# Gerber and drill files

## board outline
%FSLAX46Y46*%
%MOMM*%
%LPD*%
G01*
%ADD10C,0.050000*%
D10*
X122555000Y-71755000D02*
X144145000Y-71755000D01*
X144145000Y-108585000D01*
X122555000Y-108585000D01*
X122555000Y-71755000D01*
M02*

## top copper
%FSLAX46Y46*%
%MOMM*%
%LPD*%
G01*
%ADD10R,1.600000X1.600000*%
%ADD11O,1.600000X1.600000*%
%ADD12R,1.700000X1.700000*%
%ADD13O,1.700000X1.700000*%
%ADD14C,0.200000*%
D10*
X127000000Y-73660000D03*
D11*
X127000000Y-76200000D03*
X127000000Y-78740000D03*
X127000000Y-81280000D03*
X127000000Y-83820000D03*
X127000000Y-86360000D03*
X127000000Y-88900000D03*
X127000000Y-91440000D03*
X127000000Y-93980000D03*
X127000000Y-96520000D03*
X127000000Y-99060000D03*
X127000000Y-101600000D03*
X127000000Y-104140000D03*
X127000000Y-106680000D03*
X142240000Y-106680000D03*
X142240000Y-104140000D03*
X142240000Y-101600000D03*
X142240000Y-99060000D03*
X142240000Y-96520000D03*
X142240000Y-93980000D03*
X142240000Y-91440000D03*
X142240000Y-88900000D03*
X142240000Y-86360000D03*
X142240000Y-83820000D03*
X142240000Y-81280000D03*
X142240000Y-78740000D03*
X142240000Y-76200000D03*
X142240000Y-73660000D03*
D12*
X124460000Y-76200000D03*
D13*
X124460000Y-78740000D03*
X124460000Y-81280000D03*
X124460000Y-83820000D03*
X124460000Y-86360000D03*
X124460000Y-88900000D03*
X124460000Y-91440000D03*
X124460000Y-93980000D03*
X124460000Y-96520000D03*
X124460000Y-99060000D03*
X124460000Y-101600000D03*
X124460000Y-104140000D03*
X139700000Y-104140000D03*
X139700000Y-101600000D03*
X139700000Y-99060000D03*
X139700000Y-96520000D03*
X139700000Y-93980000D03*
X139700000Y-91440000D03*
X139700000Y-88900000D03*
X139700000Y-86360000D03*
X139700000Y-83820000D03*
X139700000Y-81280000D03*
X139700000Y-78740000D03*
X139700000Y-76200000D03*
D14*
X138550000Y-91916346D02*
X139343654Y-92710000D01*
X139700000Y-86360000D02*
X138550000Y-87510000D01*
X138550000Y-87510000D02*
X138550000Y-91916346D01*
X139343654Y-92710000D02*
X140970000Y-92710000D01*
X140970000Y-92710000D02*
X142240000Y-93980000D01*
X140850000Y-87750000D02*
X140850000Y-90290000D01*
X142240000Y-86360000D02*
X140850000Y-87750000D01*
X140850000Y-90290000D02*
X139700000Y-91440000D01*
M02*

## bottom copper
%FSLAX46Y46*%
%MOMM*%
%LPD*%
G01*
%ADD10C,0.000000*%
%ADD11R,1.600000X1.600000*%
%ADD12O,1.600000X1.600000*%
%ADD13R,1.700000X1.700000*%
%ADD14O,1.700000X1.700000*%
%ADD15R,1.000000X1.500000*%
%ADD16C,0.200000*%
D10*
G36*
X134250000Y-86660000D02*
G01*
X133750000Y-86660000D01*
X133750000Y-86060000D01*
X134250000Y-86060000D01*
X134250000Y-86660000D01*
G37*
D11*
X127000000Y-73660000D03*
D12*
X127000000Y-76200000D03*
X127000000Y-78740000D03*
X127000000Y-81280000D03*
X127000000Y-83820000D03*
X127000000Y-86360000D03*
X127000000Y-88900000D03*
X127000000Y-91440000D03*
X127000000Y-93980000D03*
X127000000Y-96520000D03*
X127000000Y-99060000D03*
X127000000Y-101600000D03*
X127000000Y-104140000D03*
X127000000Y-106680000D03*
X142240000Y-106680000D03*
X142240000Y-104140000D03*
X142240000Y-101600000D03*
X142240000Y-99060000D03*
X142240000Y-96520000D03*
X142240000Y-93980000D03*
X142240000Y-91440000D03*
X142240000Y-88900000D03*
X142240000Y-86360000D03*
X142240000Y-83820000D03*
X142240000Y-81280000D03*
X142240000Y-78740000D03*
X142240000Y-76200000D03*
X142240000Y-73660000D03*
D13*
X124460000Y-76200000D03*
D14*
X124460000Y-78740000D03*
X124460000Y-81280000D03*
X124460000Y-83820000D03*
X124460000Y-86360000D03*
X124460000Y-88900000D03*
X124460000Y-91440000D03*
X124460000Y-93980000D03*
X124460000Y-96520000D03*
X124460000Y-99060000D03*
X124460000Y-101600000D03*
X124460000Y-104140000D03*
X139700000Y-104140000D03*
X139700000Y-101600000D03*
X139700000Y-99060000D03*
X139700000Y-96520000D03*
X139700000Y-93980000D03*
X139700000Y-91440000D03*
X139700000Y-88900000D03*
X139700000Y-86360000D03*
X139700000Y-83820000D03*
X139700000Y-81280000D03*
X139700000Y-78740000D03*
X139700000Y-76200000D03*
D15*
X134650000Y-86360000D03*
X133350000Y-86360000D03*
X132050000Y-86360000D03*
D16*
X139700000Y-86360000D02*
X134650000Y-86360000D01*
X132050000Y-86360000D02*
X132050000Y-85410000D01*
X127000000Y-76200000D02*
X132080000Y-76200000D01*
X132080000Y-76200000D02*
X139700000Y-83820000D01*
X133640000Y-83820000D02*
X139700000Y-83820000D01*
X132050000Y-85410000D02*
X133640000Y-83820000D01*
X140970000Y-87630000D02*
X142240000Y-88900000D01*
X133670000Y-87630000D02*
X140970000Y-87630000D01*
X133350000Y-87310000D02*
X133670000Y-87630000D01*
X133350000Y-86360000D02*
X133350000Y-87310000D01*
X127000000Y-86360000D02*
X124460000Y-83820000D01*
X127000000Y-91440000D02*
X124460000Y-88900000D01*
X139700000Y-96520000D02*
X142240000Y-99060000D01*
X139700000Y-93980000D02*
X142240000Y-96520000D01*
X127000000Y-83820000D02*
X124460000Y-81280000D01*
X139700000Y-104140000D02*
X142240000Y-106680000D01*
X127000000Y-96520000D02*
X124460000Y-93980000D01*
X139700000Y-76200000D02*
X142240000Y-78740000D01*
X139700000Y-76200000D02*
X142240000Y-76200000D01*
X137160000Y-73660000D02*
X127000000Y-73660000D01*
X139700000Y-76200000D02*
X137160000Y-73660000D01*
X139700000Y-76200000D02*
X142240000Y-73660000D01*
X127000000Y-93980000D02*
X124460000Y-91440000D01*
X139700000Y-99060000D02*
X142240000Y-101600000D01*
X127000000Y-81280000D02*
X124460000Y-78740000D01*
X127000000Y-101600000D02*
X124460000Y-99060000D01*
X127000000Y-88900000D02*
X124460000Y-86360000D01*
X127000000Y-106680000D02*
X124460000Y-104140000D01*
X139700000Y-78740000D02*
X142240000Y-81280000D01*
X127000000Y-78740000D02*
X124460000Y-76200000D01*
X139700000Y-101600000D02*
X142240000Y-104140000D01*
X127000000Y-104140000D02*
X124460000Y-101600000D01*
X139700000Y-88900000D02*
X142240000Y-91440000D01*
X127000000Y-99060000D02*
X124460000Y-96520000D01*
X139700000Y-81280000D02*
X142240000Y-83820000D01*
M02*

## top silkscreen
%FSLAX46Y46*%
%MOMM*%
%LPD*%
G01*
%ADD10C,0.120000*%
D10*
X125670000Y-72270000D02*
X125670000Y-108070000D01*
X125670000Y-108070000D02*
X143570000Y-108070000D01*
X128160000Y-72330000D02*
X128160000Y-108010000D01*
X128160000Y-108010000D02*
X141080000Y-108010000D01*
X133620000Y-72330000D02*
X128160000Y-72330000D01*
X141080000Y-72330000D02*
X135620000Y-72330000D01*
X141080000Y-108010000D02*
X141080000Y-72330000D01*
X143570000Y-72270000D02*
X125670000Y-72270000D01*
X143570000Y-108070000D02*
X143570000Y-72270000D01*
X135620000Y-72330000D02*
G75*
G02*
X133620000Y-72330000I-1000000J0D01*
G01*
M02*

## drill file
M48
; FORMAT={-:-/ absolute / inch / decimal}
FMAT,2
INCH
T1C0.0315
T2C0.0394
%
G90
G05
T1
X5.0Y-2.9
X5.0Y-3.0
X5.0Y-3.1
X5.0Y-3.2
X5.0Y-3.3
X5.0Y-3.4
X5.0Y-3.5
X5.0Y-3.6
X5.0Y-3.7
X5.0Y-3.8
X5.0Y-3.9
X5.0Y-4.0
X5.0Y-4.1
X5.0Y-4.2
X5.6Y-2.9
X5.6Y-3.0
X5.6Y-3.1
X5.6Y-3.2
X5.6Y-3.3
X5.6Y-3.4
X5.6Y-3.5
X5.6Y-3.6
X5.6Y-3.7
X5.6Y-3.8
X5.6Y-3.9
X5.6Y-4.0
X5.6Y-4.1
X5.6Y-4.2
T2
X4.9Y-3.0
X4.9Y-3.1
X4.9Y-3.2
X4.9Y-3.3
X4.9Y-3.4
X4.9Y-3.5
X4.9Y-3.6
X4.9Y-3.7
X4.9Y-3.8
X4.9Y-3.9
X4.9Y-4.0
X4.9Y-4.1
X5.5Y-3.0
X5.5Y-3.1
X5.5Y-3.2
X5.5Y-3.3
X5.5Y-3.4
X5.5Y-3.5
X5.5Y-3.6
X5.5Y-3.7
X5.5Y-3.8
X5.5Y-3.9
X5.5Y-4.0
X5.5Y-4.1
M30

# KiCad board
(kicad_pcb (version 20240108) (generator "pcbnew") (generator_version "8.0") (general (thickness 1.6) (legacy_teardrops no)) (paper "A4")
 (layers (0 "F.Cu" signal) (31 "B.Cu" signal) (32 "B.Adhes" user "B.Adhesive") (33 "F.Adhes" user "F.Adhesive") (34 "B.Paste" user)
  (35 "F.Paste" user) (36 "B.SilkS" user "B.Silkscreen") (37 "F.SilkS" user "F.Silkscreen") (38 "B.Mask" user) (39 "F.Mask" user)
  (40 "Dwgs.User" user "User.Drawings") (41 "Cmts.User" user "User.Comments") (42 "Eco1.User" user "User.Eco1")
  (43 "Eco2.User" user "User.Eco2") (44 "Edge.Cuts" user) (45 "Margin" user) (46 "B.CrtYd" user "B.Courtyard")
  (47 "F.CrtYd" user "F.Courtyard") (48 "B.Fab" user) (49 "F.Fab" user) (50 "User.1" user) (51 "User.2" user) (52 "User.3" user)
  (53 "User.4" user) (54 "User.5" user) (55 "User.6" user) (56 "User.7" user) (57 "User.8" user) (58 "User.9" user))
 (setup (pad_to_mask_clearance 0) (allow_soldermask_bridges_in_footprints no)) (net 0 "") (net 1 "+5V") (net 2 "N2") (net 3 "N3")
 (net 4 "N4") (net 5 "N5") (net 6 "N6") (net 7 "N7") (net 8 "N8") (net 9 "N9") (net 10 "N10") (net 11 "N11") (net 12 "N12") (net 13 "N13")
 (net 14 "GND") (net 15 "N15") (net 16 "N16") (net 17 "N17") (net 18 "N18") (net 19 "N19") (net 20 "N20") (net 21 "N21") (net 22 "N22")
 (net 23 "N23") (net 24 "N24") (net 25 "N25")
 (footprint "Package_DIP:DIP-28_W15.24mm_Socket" (layer "F.Cu") (at 127 73.66)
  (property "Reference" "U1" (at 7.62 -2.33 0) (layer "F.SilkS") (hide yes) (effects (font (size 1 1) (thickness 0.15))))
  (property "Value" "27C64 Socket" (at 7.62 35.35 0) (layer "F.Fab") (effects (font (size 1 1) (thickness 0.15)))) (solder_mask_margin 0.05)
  (fp_line (start -1.33 -1.39) (end -1.33 34.41) (stroke (width 0.12) (type solid)) (layer "F.SilkS"))
  (fp_line (start -1.33 34.41) (end 16.57 34.41) (stroke (width 0.12) (type solid)) (layer "F.SilkS"))
  (fp_line (start 1.16 -1.33) (end 1.16 34.35) (stroke (width 0.12) (type solid)) (layer "F.SilkS"))
  (fp_line (start 1.16 34.35) (end 14.08 34.35) (stroke (width 0.12) (type solid)) (layer "F.SilkS"))
  (fp_line (start 6.62 -1.33) (end 1.16 -1.33) (stroke (width 0.12) (type solid)) (layer "F.SilkS"))
  (fp_line (start 14.08 -1.33) (end 8.62 -1.33) (stroke (width 0.12) (type solid)) (layer "F.SilkS"))
  (fp_line (start 14.08 34.35) (end 14.08 -1.33) (stroke (width 0.12) (type solid)) (layer "F.SilkS"))
  (fp_line (start 16.57 -1.39) (end -1.33 -1.39) (stroke (width 0.12) (type solid)) (layer "F.SilkS"))
  (fp_line (start 16.57 34.41) (end 16.57 -1.39) (stroke (width 0.12) (type solid)) (layer "F.SilkS"))
  (fp_arc (start 8.62 -1.33) (mid 7.62 -0.33) (end 6.62 -1.33) (stroke (width 0.12) (type solid)) (layer "F.SilkS"))
  (pad "1" thru_hole rect (at 0 0) (size 1.6 1.6) (drill 0.8) (layers "*.Cu" "*.Mask") (remove_unused_layers no) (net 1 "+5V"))
  (pad "2" thru_hole oval (at 0 2.54) (size 1.6 1.6) (drill 0.8) (layers "*.Cu" "*.Mask") (remove_unused_layers no) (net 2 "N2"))
  (pad "3" thru_hole oval (at 0 5.08) (size 1.6 1.6) (drill 0.8) (layers "*.Cu" "*.Mask") (remove_unused_layers no) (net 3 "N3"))
  (pad "4" thru_hole oval (at 0 7.62) (size 1.6 1.6) (drill 0.8) (layers "*.Cu" "*.Mask") (remove_unused_layers no) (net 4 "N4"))
  (pad "5" thru_hole oval (at 0 10.16) (size 1.6 1.6) (drill 0.8) (layers "*.Cu" "*.Mask") (remove_unused_layers no) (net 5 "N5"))
  (pad "6" thru_hole oval (at 0 12.7) (size 1.6 1.6) (drill 0.8) (layers "*.Cu" "*.Mask") (remove_unused_layers no) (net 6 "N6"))
  (pad "7" thru_hole oval (at 0 15.24) (size 1.6 1.6) (drill 0.8) (layers "*.Cu" "*.Mask") (remove_unused_layers no) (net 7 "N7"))
  (pad "8" thru_hole oval (at 0 17.78) (size 1.6 1.6) (drill 0.8) (layers "*.Cu" "*.Mask") (remove_unused_layers no) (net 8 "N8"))
  (pad "9" thru_hole oval (at 0 20.32) (size 1.6 1.6) (drill 0.8) (layers "*.Cu" "*.Mask") (remove_unused_layers no) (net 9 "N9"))
  (pad "10" thru_hole oval (at 0 22.86) (size 1.6 1.6) (drill 0.8) (layers "*.Cu" "*.Mask") (remove_unused_layers no) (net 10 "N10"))
  (pad "11" thru_hole oval (at 0 25.4) (size 1.6 1.6) (drill 0.8) (layers "*.Cu" "*.Mask") (remove_unused_layers no) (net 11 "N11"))
  (pad "12" thru_hole oval (at 0 27.94) (size 1.6 1.6) (drill 0.8) (layers "*.Cu" "*.Mask") (remove_unused_layers no) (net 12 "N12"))
  (pad "13" thru_hole oval (at 0 30.48) (size 1.6 1.6) (drill 0.8) (layers "*.Cu" "*.Mask") (remove_unused_layers no) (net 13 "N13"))
  (pad "14" thru_hole oval (at 0 33.02) (size 1.6 1.6) (drill 0.8) (layers "*.Cu" "*.Mask") (remove_unused_layers no) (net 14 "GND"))
  (pad "15" thru_hole oval (at 15.24 33.02) (size 1.6 1.6) (drill 0.8) (layers "*.Cu" "*.Mask") (remove_unused_layers no) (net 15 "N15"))
  (pad "16" thru_hole oval (at 15.24 30.48) (size 1.6 1.6) (drill 0.8) (layers "*.Cu" "*.Mask") (remove_unused_layers no) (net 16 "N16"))
  (pad "17" thru_hole oval (at 15.24 27.94) (size 1.6 1.6) (drill 0.8) (layers "*.Cu" "*.Mask") (remove_unused_layers no) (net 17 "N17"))
  (pad "18" thru_hole oval (at 15.24 25.4) (size 1.6 1.6) (drill 0.8) (layers "*.Cu" "*.Mask") (remove_unused_layers no) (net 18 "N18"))
  (pad "19" thru_hole oval (at 15.24 22.86) (size 1.6 1.6) (drill 0.8) (layers "*.Cu" "*.Mask") (remove_unused_layers no) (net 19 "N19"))
  (pad "20" thru_hole oval (at 15.24 20.32) (size 1.6 1.6) (drill 0.8) (layers "*.Cu" "*.Mask") (remove_unused_layers no) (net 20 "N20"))
  (pad "21" thru_hole oval (at 15.24 17.78) (size 1.6 1.6) (drill 0.8) (layers "*.Cu" "*.Mask") (remove_unused_layers no) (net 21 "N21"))
  (pad "22" thru_hole oval (at 15.24 15.24) (size 1.6 1.6) (drill 0.8) (layers "*.Cu" "*.Mask") (remove_unused_layers no) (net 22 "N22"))
  (pad "23" thru_hole oval (at 15.24 12.7) (size 1.6 1.6) (drill 0.8) (layers "*.Cu" "*.Mask") (remove_unused_layers no) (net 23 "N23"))
  (pad "24" thru_hole oval (at 15.24 10.16) (size 1.6 1.6) (drill 0.8) (layers "*.Cu" "*.Mask") (remove_unused_layers no) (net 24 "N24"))
  (pad "25" thru_hole oval (at 15.24 7.62) (size 1.6 1.6) (drill 0.8) (layers "*.Cu" "*.Mask") (remove_unused_layers no) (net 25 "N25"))
  (pad "26" thru_hole oval (at 15.24 5.08) (size 1.6 1.6) (drill 0.8) (layers "*.Cu" "*.Mask") (remove_unused_layers no) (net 1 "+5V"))
  (pad "27" thru_hole oval (at 15.24 2.54) (size 1.6 1.6) (drill 0.8) (layers "*.Cu" "*.Mask") (remove_unused_layers no) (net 1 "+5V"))
  (pad "28" thru_hole oval (at 15.24 0) (size 1.6 1.6) (drill 0.8) (layers "*.Cu" "*.Mask") (remove_unused_layers no) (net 1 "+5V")))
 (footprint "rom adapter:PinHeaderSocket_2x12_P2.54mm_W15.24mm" (layer "B.Cu") (at 139.7 76.2 180)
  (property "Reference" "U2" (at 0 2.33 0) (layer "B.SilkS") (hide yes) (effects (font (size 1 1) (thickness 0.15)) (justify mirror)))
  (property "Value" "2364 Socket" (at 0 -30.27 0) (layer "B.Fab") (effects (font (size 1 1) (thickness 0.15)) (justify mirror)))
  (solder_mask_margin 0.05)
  (pad "1" thru_hole rect (at 15.24 0 180) (size 1.7 1.7) (drill 1) (layers "*.Cu" "*.Mask") (remove_unused_layers no) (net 3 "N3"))
  (pad "2" thru_hole oval (at 15.24 -2.54 180) (size 1.7 1.7) (drill 1) (layers "*.Cu" "*.Mask") (remove_unused_layers no) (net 4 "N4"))
  (pad "3" thru_hole oval (at 15.24 -5.08 180) (size 1.7 1.7) (drill 1) (layers "*.Cu" "*.Mask") (remove_unused_layers no) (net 5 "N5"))
  (pad "4" thru_hole oval (at 15.24 -7.62 180) (size 1.7 1.7) (drill 1) (layers "*.Cu" "*.Mask") (remove_unused_layers no) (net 6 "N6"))
  (pad "5" thru_hole oval (at 15.24 -10.16 180) (size 1.7 1.7) (drill 1) (layers "*.Cu" "*.Mask") (remove_unused_layers no) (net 7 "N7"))
  (pad "6" thru_hole oval (at 15.24 -12.7 180) (size 1.7 1.7) (drill 1) (layers "*.Cu" "*.Mask") (remove_unused_layers no) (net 8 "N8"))
  (pad "7" thru_hole oval (at 15.24 -15.24 180) (size 1.7 1.7) (drill 1) (layers "*.Cu" "*.Mask") (remove_unused_layers no) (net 9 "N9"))
  (pad "8" thru_hole oval (at 15.24 -17.78 180) (size 1.7 1.7) (drill 1) (layers "*.Cu" "*.Mask") (remove_unused_layers no) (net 10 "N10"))
  (pad "9" thru_hole oval (at 15.24 -20.32 180) (size 1.7 1.7) (drill 1) (layers "*.Cu" "*.Mask") (remove_unused_layers no) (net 11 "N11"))
  (pad "10" thru_hole oval (at 15.24 -22.86 180) (size 1.7 1.7) (drill 1) (layers "*.Cu" "*.Mask") (remove_unused_layers no) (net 12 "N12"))
  (pad "11" thru_hole oval (at 15.24 -25.4 180) (size 1.7 1.7) (drill 1) (layers "*.Cu" "*.Mask") (remove_unused_layers no) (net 13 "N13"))
  (pad "12" thru_hole oval (at 15.24 -27.94 180) (size 1.7 1.7) (drill 1) (layers "*.Cu" "*.Mask") (remove_unused_layers no) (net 14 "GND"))
  (pad "13" thru_hole oval (at 0 -27.94 180) (size 1.7 1.7) (drill 1) (layers "*.Cu" "*.Mask") (remove_unused_layers no) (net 15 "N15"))
  (pad "14" thru_hole oval (at 0 -25.4 180) (size 1.7 1.7) (drill 1) (layers "*.Cu" "*.Mask") (remove_unused_layers no) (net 16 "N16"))
  (pad "15" thru_hole oval (at 0 -22.86 180) (size 1.7 1.7) (drill 1) (layers "*.Cu" "*.Mask") (remove_unused_layers no) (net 17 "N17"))
  (pad "16" thru_hole oval (at 0 -20.32 180) (size 1.7 1.7) (drill 1) (layers "*.Cu" "*.Mask") (remove_unused_layers no) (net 18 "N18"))
  (pad "17" thru_hole oval (at 0 -17.78 180) (size 1.7 1.7) (drill 1) (layers "*.Cu" "*.Mask") (remove_unused_layers no) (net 19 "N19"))
  (pad "18" thru_hole oval (at 0 -15.24 180) (size 1.7 1.7) (drill 1) (layers "*.Cu" "*.Mask") (remove_unused_layers no) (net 23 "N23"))
  (pad "19" thru_hole oval (at 0 -12.7 180) (size 1.7 1.7) (drill 1) (layers "*.Cu" "*.Mask") (remove_unused_layers no) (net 21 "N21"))
  (pad "20" thru_hole oval (at 0 -10.16 180) (size 1.7 1.7) (drill 1) (layers "*.Cu" "*.Mask") (remove_unused_layers no) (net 20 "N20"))
  (pad "21" thru_hole oval (at 0 -7.62 180) (size 1.7 1.7) (drill 1) (layers "*.Cu" "*.Mask") (remove_unused_layers no) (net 2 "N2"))
  (pad "22" thru_hole oval (at 0 -5.08 180) (size 1.7 1.7) (drill 1) (layers "*.Cu" "*.Mask") (remove_unused_layers no) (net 24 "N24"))
  (pad "23" thru_hole oval (at 0 -2.54 180) (size 1.7 1.7) (drill 1) (layers "*.Cu" "*.Mask") (remove_unused_layers no) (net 25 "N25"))
  (pad "24" thru_hole oval (at 0 0 180) (size 1.7 1.7) (drill 1) (layers "*.Cu" "*.Mask") (remove_unused_layers no) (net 1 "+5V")))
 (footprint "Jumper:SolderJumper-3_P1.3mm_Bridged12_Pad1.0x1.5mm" (layer "B.Cu") (at 133.35 86.36 180)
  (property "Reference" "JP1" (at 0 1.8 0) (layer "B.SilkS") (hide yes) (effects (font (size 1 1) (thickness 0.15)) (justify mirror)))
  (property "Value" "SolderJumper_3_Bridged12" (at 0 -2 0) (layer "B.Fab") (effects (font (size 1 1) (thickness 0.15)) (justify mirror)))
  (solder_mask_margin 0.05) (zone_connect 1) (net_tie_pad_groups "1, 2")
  (fp_poly (pts (xy -0.9 0.3) (xy -0.4 0.3) (xy -0.4 -0.3) (xy -0.9 -0.3)) (stroke (width 0) (type solid)) (fill solid) (layer "B.Cu"))
  (pad "1" smd rect (at -1.3 0 180) (size 1 1.5) (layers "B.Cu" "B.Mask") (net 20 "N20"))
  (pad "2" smd rect (at 0 0 180) (size 1 1.5) (layers "B.Cu" "B.Mask") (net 22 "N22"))
  (pad "3" smd rect (at 1.3 0 180) (size 1 1.5) (layers "B.Cu" "B.Mask") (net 2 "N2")))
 (gr_rect (start 122.555 71.755) (end 144.145 108.585) (stroke (width 0.05) (type default)) (fill none) (layer "Edge.Cuts"))
 (segment (start 138.55 91.916346) (end 139.343654 92.71) (width 0.2) (layer "F.Cu") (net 20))
 (segment (start 139.7 86.36) (end 138.55 87.51) (width 0.2) (layer "F.Cu") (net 20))
 (segment (start 138.55 87.51) (end 138.55 91.916346) (width 0.2) (layer "F.Cu") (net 20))
 (segment (start 139.343654 92.71) (end 140.97 92.71) (width 0.2) (layer "F.Cu") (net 20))
 (segment (start 140.97 92.71) (end 142.24 93.98) (width 0.2) (layer "F.Cu") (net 20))
 (segment (start 139.7 86.36) (end 134.65 86.36) (width 0.2) (layer "B.Cu") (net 20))
 (segment (start 132.05 86.36) (end 132.05 85.41) (width 0.2) (layer "B.Cu") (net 2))
 (segment (start 127 76.2) (end 132.08 76.2) (width 0.2) (layer "B.Cu") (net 2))
 (segment (start 132.08 76.2) (end 139.7 83.82) (width 0.2) (layer "B.Cu") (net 2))
 (segment (start 133.64 83.82) (end 139.7 83.82) (width 0.2) (layer "B.Cu") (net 2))
 (segment (start 132.05 85.41) (end 133.64 83.82) (width 0.2) (layer "B.Cu") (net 2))
 (segment (start 140.97 87.63) (end 142.24 88.9) (width 0.2) (layer "B.Cu") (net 22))
 (segment (start 133.67 87.63) (end 140.97 87.63) (width 0.2) (layer "B.Cu") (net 22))
 (segment (start 133.35 87.31) (end 133.67 87.63) (width 0.2) (layer "B.Cu") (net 22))
 (segment (start 133.35 86.36) (end 133.35 87.31) (width 0.2) (layer "B.Cu") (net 22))
 (segment (start 140.85 87.75) (end 140.85 90.29) (width 0.2) (layer "F.Cu") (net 23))
 (segment (start 142.24 86.36) (end 140.85 87.75) (width 0.2) (layer "F.Cu") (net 23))
 (segment (start 140.85 90.29) (end 139.7 91.44) (width 0.2) (layer "F.Cu") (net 23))
 (segment (start 127 86.36) (end 124.46 83.82) (width 0.2) (layer "B.Cu") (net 6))
 (segment (start 127 91.44) (end 124.46 88.9) (width 0.2) (layer "B.Cu") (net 8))
 (segment (start 139.7 96.52) (end 142.24 99.06) (width 0.2) (layer "B.Cu") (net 18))
 (segment (start 139.7 93.98) (end 142.24 96.52) (width 0.2) (layer "B.Cu") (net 19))
 (segment (start 127 83.82) (end 124.46 81.28) (width 0.2) (layer "B.Cu") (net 5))
 (segment (start 139.7 104.14) (end 142.24 106.68) (width 0.2) (layer "B.Cu") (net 15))
 (segment (start 127 96.52) (end 124.46 93.98) (width 0.2) (layer "B.Cu") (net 10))
 (segment (start 139.7 76.2) (end 142.24 78.74) (width 0.2) (layer "B.Cu") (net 1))
 (segment (start 139.7 76.2) (end 142.24 76.2) (width 0.2) (layer "B.Cu") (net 1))
 (segment (start 137.16 73.66) (end 127 73.66) (width 0.2) (layer "B.Cu") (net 1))
 (segment (start 139.7 76.2) (end 137.16 73.66) (width 0.2) (layer "B.Cu") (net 1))
 (segment (start 139.7 76.2) (end 142.24 73.66) (width 0.2) (layer "B.Cu") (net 1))
 (segment (start 127 93.98) (end 124.46 91.44) (width 0.2) (layer "B.Cu") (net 9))
 (segment (start 139.7 99.06) (end 142.24 101.6) (width 0.2) (layer "B.Cu") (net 17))
 (segment (start 127 81.28) (end 124.46 78.74) (width 0.2) (layer "B.Cu") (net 4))
 (segment (start 127 101.6) (end 124.46 99.06) (width 0.2) (layer "B.Cu") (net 12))
 (segment (start 127 88.9) (end 124.46 86.36) (width 0.2) (layer "B.Cu") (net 7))
 (segment (start 127 106.68) (end 124.46 104.14) (width 0.2) (layer "B.Cu") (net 14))
 (segment (start 139.7 78.74) (end 142.24 81.28) (width 0.2) (layer "B.Cu") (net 25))
 (segment (start 127 78.74) (end 124.46 76.2) (width 0.2) (layer "B.Cu") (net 3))
 (segment (start 139.7 101.6) (end 142.24 104.14) (width 0.2) (layer "B.Cu") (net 16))
 (segment (start 127 104.14) (end 124.46 101.6) (width 0.2) (layer "B.Cu") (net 13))
 (segment (start 139.7 88.9) (end 142.24 91.44) (width 0.2) (layer "B.Cu") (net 21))
 (segment (start 127 99.06) (end 124.46 96.52) (width 0.2) (layer "B.Cu") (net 11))
 (segment (start 139.7 81.28) (end 142.24 83.82) (width 0.2) (layer "B.Cu") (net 24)))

